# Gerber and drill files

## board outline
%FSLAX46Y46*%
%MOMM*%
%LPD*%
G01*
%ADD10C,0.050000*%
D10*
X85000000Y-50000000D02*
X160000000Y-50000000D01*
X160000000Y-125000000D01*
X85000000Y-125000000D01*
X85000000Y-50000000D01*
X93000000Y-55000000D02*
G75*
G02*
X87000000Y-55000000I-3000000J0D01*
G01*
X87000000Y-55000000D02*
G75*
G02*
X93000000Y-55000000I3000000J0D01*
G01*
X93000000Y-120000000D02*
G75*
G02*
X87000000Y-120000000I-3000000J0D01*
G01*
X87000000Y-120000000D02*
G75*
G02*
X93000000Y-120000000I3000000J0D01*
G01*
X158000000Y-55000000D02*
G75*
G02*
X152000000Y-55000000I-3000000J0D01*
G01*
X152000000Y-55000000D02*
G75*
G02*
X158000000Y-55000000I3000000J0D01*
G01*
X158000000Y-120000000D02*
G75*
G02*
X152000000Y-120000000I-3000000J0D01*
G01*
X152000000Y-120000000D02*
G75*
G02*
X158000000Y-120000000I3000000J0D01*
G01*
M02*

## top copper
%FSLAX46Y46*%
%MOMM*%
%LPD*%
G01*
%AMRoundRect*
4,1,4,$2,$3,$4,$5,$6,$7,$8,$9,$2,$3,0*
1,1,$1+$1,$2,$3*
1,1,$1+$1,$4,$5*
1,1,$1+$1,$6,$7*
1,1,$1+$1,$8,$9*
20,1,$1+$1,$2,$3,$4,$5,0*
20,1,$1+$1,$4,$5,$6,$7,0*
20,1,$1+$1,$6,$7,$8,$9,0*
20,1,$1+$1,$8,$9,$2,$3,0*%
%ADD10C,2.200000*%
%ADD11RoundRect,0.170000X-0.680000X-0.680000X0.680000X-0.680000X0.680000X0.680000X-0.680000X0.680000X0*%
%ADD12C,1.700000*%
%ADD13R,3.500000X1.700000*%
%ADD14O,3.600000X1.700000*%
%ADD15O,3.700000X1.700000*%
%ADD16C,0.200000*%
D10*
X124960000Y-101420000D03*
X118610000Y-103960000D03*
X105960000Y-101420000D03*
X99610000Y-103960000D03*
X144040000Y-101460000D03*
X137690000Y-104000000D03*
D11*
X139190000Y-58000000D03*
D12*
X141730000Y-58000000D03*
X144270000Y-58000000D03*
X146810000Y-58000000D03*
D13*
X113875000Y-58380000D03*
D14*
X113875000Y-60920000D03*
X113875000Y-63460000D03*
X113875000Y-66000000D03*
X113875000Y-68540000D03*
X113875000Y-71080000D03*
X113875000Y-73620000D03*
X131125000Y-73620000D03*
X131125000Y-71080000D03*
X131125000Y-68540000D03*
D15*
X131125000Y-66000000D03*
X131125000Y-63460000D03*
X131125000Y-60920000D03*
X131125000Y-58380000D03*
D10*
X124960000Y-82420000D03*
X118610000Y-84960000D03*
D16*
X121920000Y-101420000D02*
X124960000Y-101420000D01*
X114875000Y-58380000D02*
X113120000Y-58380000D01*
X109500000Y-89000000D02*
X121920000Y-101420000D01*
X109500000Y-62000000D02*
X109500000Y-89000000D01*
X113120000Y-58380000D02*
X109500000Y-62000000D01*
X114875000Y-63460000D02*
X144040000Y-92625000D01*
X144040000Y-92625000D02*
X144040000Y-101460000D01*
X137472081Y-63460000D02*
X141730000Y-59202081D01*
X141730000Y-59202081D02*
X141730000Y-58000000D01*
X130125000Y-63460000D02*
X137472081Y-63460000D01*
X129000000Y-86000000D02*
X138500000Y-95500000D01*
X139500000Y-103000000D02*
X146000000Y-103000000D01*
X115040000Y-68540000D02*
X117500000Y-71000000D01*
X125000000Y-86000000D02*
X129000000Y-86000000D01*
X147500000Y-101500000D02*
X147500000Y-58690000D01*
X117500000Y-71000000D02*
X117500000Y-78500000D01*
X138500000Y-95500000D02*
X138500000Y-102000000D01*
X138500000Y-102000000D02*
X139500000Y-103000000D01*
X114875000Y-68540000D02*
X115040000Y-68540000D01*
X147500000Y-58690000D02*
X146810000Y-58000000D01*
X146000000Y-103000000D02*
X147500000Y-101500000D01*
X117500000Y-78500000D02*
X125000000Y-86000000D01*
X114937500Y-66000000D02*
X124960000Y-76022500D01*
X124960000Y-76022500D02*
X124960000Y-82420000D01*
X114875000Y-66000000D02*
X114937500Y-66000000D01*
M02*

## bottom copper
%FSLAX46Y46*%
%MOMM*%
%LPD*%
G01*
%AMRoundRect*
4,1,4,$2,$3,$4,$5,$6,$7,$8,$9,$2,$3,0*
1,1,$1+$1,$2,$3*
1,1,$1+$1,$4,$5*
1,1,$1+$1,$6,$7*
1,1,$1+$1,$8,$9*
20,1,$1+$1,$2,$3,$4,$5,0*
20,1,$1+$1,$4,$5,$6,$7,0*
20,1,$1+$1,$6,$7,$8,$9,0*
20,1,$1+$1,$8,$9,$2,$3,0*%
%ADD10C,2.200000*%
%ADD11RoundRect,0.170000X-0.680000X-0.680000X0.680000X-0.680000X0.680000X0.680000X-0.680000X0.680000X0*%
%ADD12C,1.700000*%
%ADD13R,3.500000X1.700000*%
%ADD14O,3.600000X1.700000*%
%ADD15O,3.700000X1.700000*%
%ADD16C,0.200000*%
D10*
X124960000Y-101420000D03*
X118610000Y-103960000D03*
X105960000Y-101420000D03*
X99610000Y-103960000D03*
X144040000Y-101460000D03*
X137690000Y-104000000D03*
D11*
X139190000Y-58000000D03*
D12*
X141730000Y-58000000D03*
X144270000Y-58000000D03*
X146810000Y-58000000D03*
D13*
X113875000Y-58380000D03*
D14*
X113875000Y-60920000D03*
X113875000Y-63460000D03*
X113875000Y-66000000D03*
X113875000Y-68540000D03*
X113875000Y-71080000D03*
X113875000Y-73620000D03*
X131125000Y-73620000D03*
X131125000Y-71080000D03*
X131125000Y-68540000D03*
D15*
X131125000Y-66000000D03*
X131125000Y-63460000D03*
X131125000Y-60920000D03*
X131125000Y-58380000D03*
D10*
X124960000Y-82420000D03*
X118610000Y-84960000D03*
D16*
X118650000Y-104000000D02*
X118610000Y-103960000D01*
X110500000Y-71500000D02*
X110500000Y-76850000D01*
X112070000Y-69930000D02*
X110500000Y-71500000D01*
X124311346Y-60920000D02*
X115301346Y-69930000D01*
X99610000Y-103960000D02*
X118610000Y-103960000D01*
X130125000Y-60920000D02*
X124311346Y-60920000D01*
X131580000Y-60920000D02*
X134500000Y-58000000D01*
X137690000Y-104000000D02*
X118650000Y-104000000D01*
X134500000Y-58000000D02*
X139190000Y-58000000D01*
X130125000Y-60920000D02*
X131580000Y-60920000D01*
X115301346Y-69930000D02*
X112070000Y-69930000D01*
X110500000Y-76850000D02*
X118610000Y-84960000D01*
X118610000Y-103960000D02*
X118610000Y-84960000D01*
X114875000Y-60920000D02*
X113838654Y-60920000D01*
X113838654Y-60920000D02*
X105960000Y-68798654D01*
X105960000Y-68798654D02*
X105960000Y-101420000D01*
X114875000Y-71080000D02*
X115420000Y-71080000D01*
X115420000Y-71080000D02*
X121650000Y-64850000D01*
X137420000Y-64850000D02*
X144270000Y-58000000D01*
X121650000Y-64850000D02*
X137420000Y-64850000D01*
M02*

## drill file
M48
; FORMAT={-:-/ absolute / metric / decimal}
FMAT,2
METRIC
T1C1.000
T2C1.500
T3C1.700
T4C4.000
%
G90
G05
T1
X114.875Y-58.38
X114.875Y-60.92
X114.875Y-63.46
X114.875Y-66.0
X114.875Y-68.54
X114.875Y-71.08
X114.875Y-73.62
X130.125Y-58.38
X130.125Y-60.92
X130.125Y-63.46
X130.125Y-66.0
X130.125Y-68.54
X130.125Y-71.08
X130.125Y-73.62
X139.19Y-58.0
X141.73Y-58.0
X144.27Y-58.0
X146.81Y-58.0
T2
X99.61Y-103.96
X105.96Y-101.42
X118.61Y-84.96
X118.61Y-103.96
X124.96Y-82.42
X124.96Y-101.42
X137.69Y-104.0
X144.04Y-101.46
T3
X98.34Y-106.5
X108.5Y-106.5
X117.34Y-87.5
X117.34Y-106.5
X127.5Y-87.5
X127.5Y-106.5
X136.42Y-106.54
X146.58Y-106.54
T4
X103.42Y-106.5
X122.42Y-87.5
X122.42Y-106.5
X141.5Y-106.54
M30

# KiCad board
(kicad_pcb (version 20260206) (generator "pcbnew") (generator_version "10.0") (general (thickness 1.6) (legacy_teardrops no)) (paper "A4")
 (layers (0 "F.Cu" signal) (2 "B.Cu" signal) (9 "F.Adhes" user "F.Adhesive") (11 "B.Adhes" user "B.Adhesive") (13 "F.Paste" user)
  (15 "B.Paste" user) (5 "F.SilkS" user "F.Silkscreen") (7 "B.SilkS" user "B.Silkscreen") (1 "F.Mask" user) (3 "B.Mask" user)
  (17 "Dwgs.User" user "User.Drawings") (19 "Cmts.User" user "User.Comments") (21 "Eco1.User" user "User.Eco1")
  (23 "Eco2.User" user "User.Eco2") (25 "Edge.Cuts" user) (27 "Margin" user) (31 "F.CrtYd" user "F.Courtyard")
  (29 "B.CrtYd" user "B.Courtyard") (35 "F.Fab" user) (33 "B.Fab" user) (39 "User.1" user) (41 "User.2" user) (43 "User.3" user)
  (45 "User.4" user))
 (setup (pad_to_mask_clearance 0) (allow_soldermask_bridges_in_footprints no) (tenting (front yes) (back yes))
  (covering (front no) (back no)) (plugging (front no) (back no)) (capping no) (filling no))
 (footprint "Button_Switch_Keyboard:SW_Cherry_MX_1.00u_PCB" (layer "F.Cu") (at 124.96 101.42)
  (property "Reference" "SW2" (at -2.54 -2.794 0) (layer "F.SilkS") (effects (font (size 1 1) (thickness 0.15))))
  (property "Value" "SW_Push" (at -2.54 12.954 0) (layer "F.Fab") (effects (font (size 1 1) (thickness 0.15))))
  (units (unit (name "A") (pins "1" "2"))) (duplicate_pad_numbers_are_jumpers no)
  (pad "" np_thru_hole circle (at -7.62 5.08) (size 1.7 1.7) (drill 1.7) (layers "*.Cu" "*.Mask"))
  (pad "" np_thru_hole circle (at -2.54 5.08) (size 4 4) (drill 4) (layers "*.Cu" "*.Mask"))
  (pad "" np_thru_hole circle (at 2.54 5.08) (size 1.7 1.7) (drill 1.7) (layers "*.Cu" "*.Mask"))
  (pad "1" thru_hole circle (at 0 0) (size 2.2 2.2) (drill 1.5) (layers "*.Cu" "*.Mask") (remove_unused_layers no)
   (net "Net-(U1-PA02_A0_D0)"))
  (pad "2" thru_hole circle (at -6.35 2.54) (size 2.2 2.2) (drill 1.5) (layers "*.Cu" "*.Mask") (remove_unused_layers no) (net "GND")))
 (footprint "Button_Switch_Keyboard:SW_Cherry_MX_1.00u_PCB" (layer "F.Cu") (at 105.96 101.42)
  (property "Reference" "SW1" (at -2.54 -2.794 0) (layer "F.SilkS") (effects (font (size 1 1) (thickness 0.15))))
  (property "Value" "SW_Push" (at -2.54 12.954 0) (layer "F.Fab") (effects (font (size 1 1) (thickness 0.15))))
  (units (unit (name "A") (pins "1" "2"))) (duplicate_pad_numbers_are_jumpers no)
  (pad "" np_thru_hole circle (at -7.62 5.08) (size 1.7 1.7) (drill 1.7) (layers "*.Cu" "*.Mask"))
  (pad "" np_thru_hole circle (at -2.54 5.08) (size 4 4) (drill 4) (layers "*.Cu" "*.Mask"))
  (pad "" np_thru_hole circle (at 2.54 5.08) (size 1.7 1.7) (drill 1.7) (layers "*.Cu" "*.Mask"))
  (pad "1" thru_hole circle (at 0 0) (size 2.2 2.2) (drill 1.5) (layers "*.Cu" "*.Mask") (remove_unused_layers no)
   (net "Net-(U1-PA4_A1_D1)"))
  (pad "2" thru_hole circle (at -6.35 2.54) (size 2.2 2.2) (drill 1.5) (layers "*.Cu" "*.Mask") (remove_unused_layers no) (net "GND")))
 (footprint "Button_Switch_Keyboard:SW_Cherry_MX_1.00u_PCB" (layer "F.Cu") (at 144.04 101.46)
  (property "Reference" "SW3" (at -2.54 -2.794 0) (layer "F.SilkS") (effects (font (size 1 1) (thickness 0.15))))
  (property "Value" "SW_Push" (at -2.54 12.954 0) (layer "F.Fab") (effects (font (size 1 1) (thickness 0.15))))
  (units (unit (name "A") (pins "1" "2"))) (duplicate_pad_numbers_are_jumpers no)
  (pad "" np_thru_hole circle (at -7.62 5.08) (size 1.7 1.7) (drill 1.7) (layers "*.Cu" "*.Mask"))
  (pad "" np_thru_hole circle (at -2.54 5.08) (size 4 4) (drill 4) (layers "*.Cu" "*.Mask"))
  (pad "" np_thru_hole circle (at 2.54 5.08) (size 1.7 1.7) (drill 1.7) (layers "*.Cu" "*.Mask"))
  (pad "1" thru_hole circle (at 0 0) (size 2.2 2.2) (drill 1.5) (layers "*.Cu" "*.Mask") (remove_unused_layers no)
   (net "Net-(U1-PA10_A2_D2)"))
  (pad "2" thru_hole circle (at -6.35 2.54) (size 2.2 2.2) (drill 1.5) (layers "*.Cu" "*.Mask") (remove_unused_layers no) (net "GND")))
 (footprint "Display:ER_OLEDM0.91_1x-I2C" (layer "F.Cu") (at 139.19 58)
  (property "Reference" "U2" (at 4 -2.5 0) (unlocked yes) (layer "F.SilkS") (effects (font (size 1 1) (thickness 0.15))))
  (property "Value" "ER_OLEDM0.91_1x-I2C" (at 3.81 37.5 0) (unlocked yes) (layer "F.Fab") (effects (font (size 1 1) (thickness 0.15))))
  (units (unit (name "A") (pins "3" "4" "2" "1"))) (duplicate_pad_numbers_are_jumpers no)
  (pad "1" thru_hole roundrect (at 0 0) (size 1.7 1.7) (drill 1) (layers "*.Cu" "*.Mask") (remove_unused_layers no) (roundrect_rratio 0.1)
   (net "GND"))
  (pad "2" thru_hole circle (at 2.54 0) (size 1.7 1.7) (drill 1) (layers "*.Cu" "*.Mask") (remove_unused_layers no) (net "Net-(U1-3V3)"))
  (pad "3" thru_hole circle (at 5.08 0) (size 1.7 1.7) (drill 1) (layers "*.Cu" "*.Mask") (remove_unused_layers no)
   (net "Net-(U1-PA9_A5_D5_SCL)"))
  (pad "4" thru_hole circle (at 7.62 0) (size 1.7 1.7) (drill 1) (layers "*.Cu" "*.Mask") (remove_unused_layers no)
   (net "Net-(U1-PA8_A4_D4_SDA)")))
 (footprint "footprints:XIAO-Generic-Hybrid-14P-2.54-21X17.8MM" (layer "F.Cu") (at 122.5 66)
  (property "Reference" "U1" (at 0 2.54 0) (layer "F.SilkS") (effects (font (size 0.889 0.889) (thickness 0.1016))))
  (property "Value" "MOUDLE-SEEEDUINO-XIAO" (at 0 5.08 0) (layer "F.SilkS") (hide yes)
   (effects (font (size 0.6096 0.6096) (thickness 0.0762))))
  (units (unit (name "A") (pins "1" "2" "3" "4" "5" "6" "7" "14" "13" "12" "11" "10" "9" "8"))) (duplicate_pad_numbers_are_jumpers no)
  (pad "1" thru_hole rect (at -7.625 -7.62) (size 3.5 1.7) (drill 1 (offset -1 0)) (layers "*.Cu" "*.Mask") (remove_unused_layers no)
   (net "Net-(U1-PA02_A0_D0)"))
  (pad "2" thru_hole oval (at -7.625 -5.08) (size 3.6 1.7) (drill 1 (offset -1 0)) (layers "*.Cu" "*.Mask") (remove_unused_layers no)
   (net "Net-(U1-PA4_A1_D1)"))
  (pad "3" thru_hole oval (at -7.625 -2.54) (size 3.6 1.7) (drill 1 (offset -1 0)) (layers "*.Cu" "*.Mask") (remove_unused_layers no)
   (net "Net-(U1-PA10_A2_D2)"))
  (pad "4" thru_hole oval (at -7.625 0) (size 3.6 1.7) (drill 1 (offset -1 0)) (layers "*.Cu" "*.Mask") (remove_unused_layers no)
   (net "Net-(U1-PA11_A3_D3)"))
  (pad "5" thru_hole oval (at -7.625 2.54) (size 3.6 1.7) (drill 1 (offset -1 0)) (layers "*.Cu" "*.Mask") (remove_unused_layers no)
   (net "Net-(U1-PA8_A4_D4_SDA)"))
  (pad "6" thru_hole oval (at -7.625 5.08 180) (size 3.6 1.7) (drill 1 (offset 1 0)) (layers "*.Cu" "*.Mask") (remove_unused_layers no)
   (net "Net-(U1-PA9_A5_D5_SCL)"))
  (pad "7" thru_hole oval (at -7.625 7.62) (size 3.6 1.7) (drill 1 (offset -1 0)) (layers "*.Cu" "*.Mask") (remove_unused_layers no)
   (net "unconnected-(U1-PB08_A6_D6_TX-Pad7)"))
  (pad "8" thru_hole oval (at 7.625 7.62) (size 3.6 1.7) (drill 1 (offset 1 0)) (layers "*.Cu" "*.Mask") (remove_unused_layers no)
   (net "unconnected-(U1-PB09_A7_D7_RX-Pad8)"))
  (pad "9" thru_hole oval (at 7.625 5.08) (size 3.6 1.7) (drill 1 (offset 1 0)) (layers "*.Cu" "*.Mask") (remove_unused_layers no)
   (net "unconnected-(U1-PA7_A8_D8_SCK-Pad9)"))
  (pad "10" thru_hole oval (at 7.625 2.54) (size 3.6 1.7) (drill 1 (offset 1 0)) (layers "*.Cu" "*.Mask") (remove_unused_layers no)
   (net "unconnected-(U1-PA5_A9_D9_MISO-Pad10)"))
  (pad "11" thru_hole oval (at 7.625 0) (size 3.7 1.7) (drill 1 (offset 1 0)) (layers "*.Cu" "*.Mask") (remove_unused_layers no)
   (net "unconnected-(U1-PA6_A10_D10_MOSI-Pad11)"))
  (pad "12" thru_hole oval (at 7.625 -2.54) (size 3.7 1.7) (drill 1 (offset 1 0)) (layers "*.Cu" "*.Mask") (remove_unused_layers no)
   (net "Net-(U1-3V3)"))
  (pad "13" thru_hole oval (at 7.625 -5.08) (size 3.7 1.7) (drill 1 (offset 1 0)) (layers "*.Cu" "*.Mask") (remove_unused_layers no)
   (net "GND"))
  (pad "14" thru_hole oval (at 7.625 -7.62) (size 3.7 1.7) (drill 1 (offset 1 0)) (layers "*.Cu" "*.Mask") (remove_unused_layers no)
   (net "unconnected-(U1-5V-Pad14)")))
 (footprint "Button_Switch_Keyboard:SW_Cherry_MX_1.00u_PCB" (layer "F.Cu") (at 124.96 82.42)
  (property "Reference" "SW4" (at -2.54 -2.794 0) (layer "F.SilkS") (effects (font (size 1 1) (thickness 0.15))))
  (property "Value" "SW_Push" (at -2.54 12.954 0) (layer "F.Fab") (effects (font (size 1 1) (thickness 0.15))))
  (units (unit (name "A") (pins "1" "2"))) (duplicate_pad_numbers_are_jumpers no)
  (pad "" np_thru_hole circle (at -7.62 5.08) (size 1.7 1.7) (drill 1.7) (layers "*.Cu" "*.Mask"))
  (pad "" np_thru_hole circle (at -2.54 5.08) (size 4 4) (drill 4) (layers "*.Cu" "*.Mask"))
  (pad "" np_thru_hole circle (at 2.54 5.08) (size 1.7 1.7) (drill 1.7) (layers "*.Cu" "*.Mask"))
  (pad "1" thru_hole circle (at 0 0) (size 2.2 2.2) (drill 1.5) (layers "*.Cu" "*.Mask") (remove_unused_layers no)
   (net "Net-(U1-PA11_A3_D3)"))
  (pad "2" thru_hole circle (at -6.35 2.54) (size 2.2 2.2) (drill 1.5) (layers "*.Cu" "*.Mask") (remove_unused_layers no) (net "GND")))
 (gr_rect (start 85 50) (end 160 125) (stroke (width 0.05) (type default)) (fill no) (layer "Edge.Cuts"))
 (gr_circle (center 90 55) (end 93 55) (stroke (width 0.05) (type default)) (fill no) (layer "Edge.Cuts"))
 (gr_circle (center 90 120) (end 93 120) (stroke (width 0.05) (type default)) (fill no) (layer "Edge.Cuts"))
 (gr_circle (center 155 55) (end 158 55) (stroke (width 0.05) (type default)) (fill no) (layer "Edge.Cuts"))
 (gr_circle (center 155 120) (end 158 120) (stroke (width 0.05) (type default)) (fill no) (layer "Edge.Cuts"))
 (segment (start 121.92 101.42) (end 124.96 101.42) (width 0.2) (layer "F.Cu") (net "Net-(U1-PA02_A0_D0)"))
 (segment (start 114.875 58.38) (end 113.12 58.38) (width 0.2) (layer "F.Cu") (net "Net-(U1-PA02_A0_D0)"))
 (segment (start 109.5 89) (end 121.92 101.42) (width 0.2) (layer "F.Cu") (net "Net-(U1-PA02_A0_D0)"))
 (segment (start 109.5 62) (end 109.5 89) (width 0.2) (layer "F.Cu") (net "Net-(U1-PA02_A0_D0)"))
 (segment (start 113.12 58.38) (end 109.5 62) (width 0.2) (layer "F.Cu") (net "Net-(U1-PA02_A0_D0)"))
 (segment (start 118.65 104) (end 118.61 103.96) (width 0.2) (layer "B.Cu") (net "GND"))
 (segment (start 110.5 71.5) (end 110.5 76.85) (width 0.2) (layer "B.Cu") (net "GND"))
 (segment (start 112.07 69.93) (end 110.5 71.5) (width 0.2) (layer "B.Cu") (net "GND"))
 (segment (start 124.311346 60.92) (end 115.301346 69.93) (width 0.2) (layer "B.Cu") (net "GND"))
 (segment (start 99.61 103.96) (end 118.61 103.96) (width 0.2) (layer "B.Cu") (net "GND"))
 (segment (start 130.125 60.92) (end 124.311346 60.92) (width 0.2) (layer "B.Cu") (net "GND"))
 (segment (start 131.58 60.92) (end 134.5 58) (width 0.2) (layer "B.Cu") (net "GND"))
 (segment (start 137.69 104) (end 118.65 104) (width 0.2) (layer "B.Cu") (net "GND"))
 (segment (start 134.5 58) (end 139.19 58) (width 0.2) (layer "B.Cu") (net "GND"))
 (segment (start 130.125 60.92) (end 131.58 60.92) (width 0.2) (layer "B.Cu") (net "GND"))
 (segment (start 115.301346 69.93) (end 112.07 69.93) (width 0.2) (layer "B.Cu") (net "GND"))
 (segment (start 110.5 76.85) (end 118.61 84.96) (width 0.2) (layer "B.Cu") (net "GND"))
 (segment (start 118.61 103.96) (end 118.61 84.96) (width 0.2) (layer "B.Cu") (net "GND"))
 (segment (start 114.875 60.92) (end 113.838654 60.92) (width 0.2) (layer "B.Cu") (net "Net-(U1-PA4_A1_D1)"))
 (segment (start 113.838654 60.92) (end 105.96 68.798654) (width 0.2) (layer "B.Cu") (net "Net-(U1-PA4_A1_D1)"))
 (segment (start 105.96 68.798654) (end 105.96 101.42) (width 0.2) (layer "B.Cu") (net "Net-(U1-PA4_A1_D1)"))
 (segment (start 114.875 63.46) (end 144.04 92.625) (width 0.2) (layer "F.Cu") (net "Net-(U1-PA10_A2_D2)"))
 (segment (start 144.04 92.625) (end 144.04 101.46) (width 0.2) (layer "F.Cu") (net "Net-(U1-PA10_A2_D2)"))
 (segment (start 137.472081 63.46) (end 141.73 59.202081) (width 0.2) (layer "F.Cu") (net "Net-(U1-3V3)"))
 (segment (start 141.73 59.202081) (end 141.73 58) (width 0.2) (layer "F.Cu") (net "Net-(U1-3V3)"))
 (segment (start 130.125 63.46) (end 137.472081 63.46) (width 0.2) (layer "F.Cu") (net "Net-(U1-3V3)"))
 (segment (start 114.875 71.08) (end 115.42 71.08) (width 0.2) (layer "B.Cu") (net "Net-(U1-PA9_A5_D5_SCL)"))
 (segment (start 115.42 71.08) (end 121.65 64.85) (width 0.2) (layer "B.Cu") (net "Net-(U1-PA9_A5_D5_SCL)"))
 (segment (start 137.42 64.85) (end 144.27 58) (width 0.2) (layer "B.Cu") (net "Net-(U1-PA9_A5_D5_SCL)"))
 (segment (start 121.65 64.85) (end 137.42 64.85) (width 0.2) (layer "B.Cu") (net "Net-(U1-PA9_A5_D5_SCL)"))
 (segment (start 129 86) (end 138.5 95.5) (width 0.2) (layer "F.Cu") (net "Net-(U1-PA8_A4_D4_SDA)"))
 (segment (start 139.5 103) (end 146 103) (width 0.2) (layer "F.Cu") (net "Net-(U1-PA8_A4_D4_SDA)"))
 (segment (start 115.04 68.54) (end 117.5 71) (width 0.2) (layer "F.Cu") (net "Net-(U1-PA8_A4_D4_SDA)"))
 (segment (start 125 86) (end 129 86) (width 0.2) (layer "F.Cu") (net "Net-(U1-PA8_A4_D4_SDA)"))
 (segment (start 147.5 101.5) (end 147.5 58.69) (width 0.2) (layer "F.Cu") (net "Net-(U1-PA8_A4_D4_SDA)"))
 (segment (start 117.5 71) (end 117.5 78.5) (width 0.2) (layer "F.Cu") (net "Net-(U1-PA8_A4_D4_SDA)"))
 (segment (start 138.5 95.5) (end 138.5 102) (width 0.2) (layer "F.Cu") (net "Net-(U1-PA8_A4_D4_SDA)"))
 (segment (start 138.5 102) (end 139.5 103) (width 0.2) (layer "F.Cu") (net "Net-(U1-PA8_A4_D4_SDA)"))
 (segment (start 114.875 68.54) (end 115.04 68.54) (width 0.2) (layer "F.Cu") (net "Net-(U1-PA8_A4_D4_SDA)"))
 (segment (start 147.5 58.69) (end 146.81 58) (width 0.2) (layer "F.Cu") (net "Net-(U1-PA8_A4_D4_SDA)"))
 (segment (start 146 103) (end 147.5 101.5) (width 0.2) (layer "F.Cu") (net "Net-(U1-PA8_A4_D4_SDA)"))
 (segment (start 117.5 78.5) (end 125 86) (width 0.2) (layer "F.Cu") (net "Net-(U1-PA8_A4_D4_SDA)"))
 (segment (start 114.9375 66) (end 124.96 76.0225) (width 0.2) (layer "F.Cu") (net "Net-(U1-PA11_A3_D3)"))
 (segment (start 124.96 76.0225) (end 124.96 82.42) (width 0.2) (layer "F.Cu") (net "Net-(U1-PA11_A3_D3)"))
 (segment (start 114.875 66) (end 114.9375 66) (width 0.2) (layer "F.Cu") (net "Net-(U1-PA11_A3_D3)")))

